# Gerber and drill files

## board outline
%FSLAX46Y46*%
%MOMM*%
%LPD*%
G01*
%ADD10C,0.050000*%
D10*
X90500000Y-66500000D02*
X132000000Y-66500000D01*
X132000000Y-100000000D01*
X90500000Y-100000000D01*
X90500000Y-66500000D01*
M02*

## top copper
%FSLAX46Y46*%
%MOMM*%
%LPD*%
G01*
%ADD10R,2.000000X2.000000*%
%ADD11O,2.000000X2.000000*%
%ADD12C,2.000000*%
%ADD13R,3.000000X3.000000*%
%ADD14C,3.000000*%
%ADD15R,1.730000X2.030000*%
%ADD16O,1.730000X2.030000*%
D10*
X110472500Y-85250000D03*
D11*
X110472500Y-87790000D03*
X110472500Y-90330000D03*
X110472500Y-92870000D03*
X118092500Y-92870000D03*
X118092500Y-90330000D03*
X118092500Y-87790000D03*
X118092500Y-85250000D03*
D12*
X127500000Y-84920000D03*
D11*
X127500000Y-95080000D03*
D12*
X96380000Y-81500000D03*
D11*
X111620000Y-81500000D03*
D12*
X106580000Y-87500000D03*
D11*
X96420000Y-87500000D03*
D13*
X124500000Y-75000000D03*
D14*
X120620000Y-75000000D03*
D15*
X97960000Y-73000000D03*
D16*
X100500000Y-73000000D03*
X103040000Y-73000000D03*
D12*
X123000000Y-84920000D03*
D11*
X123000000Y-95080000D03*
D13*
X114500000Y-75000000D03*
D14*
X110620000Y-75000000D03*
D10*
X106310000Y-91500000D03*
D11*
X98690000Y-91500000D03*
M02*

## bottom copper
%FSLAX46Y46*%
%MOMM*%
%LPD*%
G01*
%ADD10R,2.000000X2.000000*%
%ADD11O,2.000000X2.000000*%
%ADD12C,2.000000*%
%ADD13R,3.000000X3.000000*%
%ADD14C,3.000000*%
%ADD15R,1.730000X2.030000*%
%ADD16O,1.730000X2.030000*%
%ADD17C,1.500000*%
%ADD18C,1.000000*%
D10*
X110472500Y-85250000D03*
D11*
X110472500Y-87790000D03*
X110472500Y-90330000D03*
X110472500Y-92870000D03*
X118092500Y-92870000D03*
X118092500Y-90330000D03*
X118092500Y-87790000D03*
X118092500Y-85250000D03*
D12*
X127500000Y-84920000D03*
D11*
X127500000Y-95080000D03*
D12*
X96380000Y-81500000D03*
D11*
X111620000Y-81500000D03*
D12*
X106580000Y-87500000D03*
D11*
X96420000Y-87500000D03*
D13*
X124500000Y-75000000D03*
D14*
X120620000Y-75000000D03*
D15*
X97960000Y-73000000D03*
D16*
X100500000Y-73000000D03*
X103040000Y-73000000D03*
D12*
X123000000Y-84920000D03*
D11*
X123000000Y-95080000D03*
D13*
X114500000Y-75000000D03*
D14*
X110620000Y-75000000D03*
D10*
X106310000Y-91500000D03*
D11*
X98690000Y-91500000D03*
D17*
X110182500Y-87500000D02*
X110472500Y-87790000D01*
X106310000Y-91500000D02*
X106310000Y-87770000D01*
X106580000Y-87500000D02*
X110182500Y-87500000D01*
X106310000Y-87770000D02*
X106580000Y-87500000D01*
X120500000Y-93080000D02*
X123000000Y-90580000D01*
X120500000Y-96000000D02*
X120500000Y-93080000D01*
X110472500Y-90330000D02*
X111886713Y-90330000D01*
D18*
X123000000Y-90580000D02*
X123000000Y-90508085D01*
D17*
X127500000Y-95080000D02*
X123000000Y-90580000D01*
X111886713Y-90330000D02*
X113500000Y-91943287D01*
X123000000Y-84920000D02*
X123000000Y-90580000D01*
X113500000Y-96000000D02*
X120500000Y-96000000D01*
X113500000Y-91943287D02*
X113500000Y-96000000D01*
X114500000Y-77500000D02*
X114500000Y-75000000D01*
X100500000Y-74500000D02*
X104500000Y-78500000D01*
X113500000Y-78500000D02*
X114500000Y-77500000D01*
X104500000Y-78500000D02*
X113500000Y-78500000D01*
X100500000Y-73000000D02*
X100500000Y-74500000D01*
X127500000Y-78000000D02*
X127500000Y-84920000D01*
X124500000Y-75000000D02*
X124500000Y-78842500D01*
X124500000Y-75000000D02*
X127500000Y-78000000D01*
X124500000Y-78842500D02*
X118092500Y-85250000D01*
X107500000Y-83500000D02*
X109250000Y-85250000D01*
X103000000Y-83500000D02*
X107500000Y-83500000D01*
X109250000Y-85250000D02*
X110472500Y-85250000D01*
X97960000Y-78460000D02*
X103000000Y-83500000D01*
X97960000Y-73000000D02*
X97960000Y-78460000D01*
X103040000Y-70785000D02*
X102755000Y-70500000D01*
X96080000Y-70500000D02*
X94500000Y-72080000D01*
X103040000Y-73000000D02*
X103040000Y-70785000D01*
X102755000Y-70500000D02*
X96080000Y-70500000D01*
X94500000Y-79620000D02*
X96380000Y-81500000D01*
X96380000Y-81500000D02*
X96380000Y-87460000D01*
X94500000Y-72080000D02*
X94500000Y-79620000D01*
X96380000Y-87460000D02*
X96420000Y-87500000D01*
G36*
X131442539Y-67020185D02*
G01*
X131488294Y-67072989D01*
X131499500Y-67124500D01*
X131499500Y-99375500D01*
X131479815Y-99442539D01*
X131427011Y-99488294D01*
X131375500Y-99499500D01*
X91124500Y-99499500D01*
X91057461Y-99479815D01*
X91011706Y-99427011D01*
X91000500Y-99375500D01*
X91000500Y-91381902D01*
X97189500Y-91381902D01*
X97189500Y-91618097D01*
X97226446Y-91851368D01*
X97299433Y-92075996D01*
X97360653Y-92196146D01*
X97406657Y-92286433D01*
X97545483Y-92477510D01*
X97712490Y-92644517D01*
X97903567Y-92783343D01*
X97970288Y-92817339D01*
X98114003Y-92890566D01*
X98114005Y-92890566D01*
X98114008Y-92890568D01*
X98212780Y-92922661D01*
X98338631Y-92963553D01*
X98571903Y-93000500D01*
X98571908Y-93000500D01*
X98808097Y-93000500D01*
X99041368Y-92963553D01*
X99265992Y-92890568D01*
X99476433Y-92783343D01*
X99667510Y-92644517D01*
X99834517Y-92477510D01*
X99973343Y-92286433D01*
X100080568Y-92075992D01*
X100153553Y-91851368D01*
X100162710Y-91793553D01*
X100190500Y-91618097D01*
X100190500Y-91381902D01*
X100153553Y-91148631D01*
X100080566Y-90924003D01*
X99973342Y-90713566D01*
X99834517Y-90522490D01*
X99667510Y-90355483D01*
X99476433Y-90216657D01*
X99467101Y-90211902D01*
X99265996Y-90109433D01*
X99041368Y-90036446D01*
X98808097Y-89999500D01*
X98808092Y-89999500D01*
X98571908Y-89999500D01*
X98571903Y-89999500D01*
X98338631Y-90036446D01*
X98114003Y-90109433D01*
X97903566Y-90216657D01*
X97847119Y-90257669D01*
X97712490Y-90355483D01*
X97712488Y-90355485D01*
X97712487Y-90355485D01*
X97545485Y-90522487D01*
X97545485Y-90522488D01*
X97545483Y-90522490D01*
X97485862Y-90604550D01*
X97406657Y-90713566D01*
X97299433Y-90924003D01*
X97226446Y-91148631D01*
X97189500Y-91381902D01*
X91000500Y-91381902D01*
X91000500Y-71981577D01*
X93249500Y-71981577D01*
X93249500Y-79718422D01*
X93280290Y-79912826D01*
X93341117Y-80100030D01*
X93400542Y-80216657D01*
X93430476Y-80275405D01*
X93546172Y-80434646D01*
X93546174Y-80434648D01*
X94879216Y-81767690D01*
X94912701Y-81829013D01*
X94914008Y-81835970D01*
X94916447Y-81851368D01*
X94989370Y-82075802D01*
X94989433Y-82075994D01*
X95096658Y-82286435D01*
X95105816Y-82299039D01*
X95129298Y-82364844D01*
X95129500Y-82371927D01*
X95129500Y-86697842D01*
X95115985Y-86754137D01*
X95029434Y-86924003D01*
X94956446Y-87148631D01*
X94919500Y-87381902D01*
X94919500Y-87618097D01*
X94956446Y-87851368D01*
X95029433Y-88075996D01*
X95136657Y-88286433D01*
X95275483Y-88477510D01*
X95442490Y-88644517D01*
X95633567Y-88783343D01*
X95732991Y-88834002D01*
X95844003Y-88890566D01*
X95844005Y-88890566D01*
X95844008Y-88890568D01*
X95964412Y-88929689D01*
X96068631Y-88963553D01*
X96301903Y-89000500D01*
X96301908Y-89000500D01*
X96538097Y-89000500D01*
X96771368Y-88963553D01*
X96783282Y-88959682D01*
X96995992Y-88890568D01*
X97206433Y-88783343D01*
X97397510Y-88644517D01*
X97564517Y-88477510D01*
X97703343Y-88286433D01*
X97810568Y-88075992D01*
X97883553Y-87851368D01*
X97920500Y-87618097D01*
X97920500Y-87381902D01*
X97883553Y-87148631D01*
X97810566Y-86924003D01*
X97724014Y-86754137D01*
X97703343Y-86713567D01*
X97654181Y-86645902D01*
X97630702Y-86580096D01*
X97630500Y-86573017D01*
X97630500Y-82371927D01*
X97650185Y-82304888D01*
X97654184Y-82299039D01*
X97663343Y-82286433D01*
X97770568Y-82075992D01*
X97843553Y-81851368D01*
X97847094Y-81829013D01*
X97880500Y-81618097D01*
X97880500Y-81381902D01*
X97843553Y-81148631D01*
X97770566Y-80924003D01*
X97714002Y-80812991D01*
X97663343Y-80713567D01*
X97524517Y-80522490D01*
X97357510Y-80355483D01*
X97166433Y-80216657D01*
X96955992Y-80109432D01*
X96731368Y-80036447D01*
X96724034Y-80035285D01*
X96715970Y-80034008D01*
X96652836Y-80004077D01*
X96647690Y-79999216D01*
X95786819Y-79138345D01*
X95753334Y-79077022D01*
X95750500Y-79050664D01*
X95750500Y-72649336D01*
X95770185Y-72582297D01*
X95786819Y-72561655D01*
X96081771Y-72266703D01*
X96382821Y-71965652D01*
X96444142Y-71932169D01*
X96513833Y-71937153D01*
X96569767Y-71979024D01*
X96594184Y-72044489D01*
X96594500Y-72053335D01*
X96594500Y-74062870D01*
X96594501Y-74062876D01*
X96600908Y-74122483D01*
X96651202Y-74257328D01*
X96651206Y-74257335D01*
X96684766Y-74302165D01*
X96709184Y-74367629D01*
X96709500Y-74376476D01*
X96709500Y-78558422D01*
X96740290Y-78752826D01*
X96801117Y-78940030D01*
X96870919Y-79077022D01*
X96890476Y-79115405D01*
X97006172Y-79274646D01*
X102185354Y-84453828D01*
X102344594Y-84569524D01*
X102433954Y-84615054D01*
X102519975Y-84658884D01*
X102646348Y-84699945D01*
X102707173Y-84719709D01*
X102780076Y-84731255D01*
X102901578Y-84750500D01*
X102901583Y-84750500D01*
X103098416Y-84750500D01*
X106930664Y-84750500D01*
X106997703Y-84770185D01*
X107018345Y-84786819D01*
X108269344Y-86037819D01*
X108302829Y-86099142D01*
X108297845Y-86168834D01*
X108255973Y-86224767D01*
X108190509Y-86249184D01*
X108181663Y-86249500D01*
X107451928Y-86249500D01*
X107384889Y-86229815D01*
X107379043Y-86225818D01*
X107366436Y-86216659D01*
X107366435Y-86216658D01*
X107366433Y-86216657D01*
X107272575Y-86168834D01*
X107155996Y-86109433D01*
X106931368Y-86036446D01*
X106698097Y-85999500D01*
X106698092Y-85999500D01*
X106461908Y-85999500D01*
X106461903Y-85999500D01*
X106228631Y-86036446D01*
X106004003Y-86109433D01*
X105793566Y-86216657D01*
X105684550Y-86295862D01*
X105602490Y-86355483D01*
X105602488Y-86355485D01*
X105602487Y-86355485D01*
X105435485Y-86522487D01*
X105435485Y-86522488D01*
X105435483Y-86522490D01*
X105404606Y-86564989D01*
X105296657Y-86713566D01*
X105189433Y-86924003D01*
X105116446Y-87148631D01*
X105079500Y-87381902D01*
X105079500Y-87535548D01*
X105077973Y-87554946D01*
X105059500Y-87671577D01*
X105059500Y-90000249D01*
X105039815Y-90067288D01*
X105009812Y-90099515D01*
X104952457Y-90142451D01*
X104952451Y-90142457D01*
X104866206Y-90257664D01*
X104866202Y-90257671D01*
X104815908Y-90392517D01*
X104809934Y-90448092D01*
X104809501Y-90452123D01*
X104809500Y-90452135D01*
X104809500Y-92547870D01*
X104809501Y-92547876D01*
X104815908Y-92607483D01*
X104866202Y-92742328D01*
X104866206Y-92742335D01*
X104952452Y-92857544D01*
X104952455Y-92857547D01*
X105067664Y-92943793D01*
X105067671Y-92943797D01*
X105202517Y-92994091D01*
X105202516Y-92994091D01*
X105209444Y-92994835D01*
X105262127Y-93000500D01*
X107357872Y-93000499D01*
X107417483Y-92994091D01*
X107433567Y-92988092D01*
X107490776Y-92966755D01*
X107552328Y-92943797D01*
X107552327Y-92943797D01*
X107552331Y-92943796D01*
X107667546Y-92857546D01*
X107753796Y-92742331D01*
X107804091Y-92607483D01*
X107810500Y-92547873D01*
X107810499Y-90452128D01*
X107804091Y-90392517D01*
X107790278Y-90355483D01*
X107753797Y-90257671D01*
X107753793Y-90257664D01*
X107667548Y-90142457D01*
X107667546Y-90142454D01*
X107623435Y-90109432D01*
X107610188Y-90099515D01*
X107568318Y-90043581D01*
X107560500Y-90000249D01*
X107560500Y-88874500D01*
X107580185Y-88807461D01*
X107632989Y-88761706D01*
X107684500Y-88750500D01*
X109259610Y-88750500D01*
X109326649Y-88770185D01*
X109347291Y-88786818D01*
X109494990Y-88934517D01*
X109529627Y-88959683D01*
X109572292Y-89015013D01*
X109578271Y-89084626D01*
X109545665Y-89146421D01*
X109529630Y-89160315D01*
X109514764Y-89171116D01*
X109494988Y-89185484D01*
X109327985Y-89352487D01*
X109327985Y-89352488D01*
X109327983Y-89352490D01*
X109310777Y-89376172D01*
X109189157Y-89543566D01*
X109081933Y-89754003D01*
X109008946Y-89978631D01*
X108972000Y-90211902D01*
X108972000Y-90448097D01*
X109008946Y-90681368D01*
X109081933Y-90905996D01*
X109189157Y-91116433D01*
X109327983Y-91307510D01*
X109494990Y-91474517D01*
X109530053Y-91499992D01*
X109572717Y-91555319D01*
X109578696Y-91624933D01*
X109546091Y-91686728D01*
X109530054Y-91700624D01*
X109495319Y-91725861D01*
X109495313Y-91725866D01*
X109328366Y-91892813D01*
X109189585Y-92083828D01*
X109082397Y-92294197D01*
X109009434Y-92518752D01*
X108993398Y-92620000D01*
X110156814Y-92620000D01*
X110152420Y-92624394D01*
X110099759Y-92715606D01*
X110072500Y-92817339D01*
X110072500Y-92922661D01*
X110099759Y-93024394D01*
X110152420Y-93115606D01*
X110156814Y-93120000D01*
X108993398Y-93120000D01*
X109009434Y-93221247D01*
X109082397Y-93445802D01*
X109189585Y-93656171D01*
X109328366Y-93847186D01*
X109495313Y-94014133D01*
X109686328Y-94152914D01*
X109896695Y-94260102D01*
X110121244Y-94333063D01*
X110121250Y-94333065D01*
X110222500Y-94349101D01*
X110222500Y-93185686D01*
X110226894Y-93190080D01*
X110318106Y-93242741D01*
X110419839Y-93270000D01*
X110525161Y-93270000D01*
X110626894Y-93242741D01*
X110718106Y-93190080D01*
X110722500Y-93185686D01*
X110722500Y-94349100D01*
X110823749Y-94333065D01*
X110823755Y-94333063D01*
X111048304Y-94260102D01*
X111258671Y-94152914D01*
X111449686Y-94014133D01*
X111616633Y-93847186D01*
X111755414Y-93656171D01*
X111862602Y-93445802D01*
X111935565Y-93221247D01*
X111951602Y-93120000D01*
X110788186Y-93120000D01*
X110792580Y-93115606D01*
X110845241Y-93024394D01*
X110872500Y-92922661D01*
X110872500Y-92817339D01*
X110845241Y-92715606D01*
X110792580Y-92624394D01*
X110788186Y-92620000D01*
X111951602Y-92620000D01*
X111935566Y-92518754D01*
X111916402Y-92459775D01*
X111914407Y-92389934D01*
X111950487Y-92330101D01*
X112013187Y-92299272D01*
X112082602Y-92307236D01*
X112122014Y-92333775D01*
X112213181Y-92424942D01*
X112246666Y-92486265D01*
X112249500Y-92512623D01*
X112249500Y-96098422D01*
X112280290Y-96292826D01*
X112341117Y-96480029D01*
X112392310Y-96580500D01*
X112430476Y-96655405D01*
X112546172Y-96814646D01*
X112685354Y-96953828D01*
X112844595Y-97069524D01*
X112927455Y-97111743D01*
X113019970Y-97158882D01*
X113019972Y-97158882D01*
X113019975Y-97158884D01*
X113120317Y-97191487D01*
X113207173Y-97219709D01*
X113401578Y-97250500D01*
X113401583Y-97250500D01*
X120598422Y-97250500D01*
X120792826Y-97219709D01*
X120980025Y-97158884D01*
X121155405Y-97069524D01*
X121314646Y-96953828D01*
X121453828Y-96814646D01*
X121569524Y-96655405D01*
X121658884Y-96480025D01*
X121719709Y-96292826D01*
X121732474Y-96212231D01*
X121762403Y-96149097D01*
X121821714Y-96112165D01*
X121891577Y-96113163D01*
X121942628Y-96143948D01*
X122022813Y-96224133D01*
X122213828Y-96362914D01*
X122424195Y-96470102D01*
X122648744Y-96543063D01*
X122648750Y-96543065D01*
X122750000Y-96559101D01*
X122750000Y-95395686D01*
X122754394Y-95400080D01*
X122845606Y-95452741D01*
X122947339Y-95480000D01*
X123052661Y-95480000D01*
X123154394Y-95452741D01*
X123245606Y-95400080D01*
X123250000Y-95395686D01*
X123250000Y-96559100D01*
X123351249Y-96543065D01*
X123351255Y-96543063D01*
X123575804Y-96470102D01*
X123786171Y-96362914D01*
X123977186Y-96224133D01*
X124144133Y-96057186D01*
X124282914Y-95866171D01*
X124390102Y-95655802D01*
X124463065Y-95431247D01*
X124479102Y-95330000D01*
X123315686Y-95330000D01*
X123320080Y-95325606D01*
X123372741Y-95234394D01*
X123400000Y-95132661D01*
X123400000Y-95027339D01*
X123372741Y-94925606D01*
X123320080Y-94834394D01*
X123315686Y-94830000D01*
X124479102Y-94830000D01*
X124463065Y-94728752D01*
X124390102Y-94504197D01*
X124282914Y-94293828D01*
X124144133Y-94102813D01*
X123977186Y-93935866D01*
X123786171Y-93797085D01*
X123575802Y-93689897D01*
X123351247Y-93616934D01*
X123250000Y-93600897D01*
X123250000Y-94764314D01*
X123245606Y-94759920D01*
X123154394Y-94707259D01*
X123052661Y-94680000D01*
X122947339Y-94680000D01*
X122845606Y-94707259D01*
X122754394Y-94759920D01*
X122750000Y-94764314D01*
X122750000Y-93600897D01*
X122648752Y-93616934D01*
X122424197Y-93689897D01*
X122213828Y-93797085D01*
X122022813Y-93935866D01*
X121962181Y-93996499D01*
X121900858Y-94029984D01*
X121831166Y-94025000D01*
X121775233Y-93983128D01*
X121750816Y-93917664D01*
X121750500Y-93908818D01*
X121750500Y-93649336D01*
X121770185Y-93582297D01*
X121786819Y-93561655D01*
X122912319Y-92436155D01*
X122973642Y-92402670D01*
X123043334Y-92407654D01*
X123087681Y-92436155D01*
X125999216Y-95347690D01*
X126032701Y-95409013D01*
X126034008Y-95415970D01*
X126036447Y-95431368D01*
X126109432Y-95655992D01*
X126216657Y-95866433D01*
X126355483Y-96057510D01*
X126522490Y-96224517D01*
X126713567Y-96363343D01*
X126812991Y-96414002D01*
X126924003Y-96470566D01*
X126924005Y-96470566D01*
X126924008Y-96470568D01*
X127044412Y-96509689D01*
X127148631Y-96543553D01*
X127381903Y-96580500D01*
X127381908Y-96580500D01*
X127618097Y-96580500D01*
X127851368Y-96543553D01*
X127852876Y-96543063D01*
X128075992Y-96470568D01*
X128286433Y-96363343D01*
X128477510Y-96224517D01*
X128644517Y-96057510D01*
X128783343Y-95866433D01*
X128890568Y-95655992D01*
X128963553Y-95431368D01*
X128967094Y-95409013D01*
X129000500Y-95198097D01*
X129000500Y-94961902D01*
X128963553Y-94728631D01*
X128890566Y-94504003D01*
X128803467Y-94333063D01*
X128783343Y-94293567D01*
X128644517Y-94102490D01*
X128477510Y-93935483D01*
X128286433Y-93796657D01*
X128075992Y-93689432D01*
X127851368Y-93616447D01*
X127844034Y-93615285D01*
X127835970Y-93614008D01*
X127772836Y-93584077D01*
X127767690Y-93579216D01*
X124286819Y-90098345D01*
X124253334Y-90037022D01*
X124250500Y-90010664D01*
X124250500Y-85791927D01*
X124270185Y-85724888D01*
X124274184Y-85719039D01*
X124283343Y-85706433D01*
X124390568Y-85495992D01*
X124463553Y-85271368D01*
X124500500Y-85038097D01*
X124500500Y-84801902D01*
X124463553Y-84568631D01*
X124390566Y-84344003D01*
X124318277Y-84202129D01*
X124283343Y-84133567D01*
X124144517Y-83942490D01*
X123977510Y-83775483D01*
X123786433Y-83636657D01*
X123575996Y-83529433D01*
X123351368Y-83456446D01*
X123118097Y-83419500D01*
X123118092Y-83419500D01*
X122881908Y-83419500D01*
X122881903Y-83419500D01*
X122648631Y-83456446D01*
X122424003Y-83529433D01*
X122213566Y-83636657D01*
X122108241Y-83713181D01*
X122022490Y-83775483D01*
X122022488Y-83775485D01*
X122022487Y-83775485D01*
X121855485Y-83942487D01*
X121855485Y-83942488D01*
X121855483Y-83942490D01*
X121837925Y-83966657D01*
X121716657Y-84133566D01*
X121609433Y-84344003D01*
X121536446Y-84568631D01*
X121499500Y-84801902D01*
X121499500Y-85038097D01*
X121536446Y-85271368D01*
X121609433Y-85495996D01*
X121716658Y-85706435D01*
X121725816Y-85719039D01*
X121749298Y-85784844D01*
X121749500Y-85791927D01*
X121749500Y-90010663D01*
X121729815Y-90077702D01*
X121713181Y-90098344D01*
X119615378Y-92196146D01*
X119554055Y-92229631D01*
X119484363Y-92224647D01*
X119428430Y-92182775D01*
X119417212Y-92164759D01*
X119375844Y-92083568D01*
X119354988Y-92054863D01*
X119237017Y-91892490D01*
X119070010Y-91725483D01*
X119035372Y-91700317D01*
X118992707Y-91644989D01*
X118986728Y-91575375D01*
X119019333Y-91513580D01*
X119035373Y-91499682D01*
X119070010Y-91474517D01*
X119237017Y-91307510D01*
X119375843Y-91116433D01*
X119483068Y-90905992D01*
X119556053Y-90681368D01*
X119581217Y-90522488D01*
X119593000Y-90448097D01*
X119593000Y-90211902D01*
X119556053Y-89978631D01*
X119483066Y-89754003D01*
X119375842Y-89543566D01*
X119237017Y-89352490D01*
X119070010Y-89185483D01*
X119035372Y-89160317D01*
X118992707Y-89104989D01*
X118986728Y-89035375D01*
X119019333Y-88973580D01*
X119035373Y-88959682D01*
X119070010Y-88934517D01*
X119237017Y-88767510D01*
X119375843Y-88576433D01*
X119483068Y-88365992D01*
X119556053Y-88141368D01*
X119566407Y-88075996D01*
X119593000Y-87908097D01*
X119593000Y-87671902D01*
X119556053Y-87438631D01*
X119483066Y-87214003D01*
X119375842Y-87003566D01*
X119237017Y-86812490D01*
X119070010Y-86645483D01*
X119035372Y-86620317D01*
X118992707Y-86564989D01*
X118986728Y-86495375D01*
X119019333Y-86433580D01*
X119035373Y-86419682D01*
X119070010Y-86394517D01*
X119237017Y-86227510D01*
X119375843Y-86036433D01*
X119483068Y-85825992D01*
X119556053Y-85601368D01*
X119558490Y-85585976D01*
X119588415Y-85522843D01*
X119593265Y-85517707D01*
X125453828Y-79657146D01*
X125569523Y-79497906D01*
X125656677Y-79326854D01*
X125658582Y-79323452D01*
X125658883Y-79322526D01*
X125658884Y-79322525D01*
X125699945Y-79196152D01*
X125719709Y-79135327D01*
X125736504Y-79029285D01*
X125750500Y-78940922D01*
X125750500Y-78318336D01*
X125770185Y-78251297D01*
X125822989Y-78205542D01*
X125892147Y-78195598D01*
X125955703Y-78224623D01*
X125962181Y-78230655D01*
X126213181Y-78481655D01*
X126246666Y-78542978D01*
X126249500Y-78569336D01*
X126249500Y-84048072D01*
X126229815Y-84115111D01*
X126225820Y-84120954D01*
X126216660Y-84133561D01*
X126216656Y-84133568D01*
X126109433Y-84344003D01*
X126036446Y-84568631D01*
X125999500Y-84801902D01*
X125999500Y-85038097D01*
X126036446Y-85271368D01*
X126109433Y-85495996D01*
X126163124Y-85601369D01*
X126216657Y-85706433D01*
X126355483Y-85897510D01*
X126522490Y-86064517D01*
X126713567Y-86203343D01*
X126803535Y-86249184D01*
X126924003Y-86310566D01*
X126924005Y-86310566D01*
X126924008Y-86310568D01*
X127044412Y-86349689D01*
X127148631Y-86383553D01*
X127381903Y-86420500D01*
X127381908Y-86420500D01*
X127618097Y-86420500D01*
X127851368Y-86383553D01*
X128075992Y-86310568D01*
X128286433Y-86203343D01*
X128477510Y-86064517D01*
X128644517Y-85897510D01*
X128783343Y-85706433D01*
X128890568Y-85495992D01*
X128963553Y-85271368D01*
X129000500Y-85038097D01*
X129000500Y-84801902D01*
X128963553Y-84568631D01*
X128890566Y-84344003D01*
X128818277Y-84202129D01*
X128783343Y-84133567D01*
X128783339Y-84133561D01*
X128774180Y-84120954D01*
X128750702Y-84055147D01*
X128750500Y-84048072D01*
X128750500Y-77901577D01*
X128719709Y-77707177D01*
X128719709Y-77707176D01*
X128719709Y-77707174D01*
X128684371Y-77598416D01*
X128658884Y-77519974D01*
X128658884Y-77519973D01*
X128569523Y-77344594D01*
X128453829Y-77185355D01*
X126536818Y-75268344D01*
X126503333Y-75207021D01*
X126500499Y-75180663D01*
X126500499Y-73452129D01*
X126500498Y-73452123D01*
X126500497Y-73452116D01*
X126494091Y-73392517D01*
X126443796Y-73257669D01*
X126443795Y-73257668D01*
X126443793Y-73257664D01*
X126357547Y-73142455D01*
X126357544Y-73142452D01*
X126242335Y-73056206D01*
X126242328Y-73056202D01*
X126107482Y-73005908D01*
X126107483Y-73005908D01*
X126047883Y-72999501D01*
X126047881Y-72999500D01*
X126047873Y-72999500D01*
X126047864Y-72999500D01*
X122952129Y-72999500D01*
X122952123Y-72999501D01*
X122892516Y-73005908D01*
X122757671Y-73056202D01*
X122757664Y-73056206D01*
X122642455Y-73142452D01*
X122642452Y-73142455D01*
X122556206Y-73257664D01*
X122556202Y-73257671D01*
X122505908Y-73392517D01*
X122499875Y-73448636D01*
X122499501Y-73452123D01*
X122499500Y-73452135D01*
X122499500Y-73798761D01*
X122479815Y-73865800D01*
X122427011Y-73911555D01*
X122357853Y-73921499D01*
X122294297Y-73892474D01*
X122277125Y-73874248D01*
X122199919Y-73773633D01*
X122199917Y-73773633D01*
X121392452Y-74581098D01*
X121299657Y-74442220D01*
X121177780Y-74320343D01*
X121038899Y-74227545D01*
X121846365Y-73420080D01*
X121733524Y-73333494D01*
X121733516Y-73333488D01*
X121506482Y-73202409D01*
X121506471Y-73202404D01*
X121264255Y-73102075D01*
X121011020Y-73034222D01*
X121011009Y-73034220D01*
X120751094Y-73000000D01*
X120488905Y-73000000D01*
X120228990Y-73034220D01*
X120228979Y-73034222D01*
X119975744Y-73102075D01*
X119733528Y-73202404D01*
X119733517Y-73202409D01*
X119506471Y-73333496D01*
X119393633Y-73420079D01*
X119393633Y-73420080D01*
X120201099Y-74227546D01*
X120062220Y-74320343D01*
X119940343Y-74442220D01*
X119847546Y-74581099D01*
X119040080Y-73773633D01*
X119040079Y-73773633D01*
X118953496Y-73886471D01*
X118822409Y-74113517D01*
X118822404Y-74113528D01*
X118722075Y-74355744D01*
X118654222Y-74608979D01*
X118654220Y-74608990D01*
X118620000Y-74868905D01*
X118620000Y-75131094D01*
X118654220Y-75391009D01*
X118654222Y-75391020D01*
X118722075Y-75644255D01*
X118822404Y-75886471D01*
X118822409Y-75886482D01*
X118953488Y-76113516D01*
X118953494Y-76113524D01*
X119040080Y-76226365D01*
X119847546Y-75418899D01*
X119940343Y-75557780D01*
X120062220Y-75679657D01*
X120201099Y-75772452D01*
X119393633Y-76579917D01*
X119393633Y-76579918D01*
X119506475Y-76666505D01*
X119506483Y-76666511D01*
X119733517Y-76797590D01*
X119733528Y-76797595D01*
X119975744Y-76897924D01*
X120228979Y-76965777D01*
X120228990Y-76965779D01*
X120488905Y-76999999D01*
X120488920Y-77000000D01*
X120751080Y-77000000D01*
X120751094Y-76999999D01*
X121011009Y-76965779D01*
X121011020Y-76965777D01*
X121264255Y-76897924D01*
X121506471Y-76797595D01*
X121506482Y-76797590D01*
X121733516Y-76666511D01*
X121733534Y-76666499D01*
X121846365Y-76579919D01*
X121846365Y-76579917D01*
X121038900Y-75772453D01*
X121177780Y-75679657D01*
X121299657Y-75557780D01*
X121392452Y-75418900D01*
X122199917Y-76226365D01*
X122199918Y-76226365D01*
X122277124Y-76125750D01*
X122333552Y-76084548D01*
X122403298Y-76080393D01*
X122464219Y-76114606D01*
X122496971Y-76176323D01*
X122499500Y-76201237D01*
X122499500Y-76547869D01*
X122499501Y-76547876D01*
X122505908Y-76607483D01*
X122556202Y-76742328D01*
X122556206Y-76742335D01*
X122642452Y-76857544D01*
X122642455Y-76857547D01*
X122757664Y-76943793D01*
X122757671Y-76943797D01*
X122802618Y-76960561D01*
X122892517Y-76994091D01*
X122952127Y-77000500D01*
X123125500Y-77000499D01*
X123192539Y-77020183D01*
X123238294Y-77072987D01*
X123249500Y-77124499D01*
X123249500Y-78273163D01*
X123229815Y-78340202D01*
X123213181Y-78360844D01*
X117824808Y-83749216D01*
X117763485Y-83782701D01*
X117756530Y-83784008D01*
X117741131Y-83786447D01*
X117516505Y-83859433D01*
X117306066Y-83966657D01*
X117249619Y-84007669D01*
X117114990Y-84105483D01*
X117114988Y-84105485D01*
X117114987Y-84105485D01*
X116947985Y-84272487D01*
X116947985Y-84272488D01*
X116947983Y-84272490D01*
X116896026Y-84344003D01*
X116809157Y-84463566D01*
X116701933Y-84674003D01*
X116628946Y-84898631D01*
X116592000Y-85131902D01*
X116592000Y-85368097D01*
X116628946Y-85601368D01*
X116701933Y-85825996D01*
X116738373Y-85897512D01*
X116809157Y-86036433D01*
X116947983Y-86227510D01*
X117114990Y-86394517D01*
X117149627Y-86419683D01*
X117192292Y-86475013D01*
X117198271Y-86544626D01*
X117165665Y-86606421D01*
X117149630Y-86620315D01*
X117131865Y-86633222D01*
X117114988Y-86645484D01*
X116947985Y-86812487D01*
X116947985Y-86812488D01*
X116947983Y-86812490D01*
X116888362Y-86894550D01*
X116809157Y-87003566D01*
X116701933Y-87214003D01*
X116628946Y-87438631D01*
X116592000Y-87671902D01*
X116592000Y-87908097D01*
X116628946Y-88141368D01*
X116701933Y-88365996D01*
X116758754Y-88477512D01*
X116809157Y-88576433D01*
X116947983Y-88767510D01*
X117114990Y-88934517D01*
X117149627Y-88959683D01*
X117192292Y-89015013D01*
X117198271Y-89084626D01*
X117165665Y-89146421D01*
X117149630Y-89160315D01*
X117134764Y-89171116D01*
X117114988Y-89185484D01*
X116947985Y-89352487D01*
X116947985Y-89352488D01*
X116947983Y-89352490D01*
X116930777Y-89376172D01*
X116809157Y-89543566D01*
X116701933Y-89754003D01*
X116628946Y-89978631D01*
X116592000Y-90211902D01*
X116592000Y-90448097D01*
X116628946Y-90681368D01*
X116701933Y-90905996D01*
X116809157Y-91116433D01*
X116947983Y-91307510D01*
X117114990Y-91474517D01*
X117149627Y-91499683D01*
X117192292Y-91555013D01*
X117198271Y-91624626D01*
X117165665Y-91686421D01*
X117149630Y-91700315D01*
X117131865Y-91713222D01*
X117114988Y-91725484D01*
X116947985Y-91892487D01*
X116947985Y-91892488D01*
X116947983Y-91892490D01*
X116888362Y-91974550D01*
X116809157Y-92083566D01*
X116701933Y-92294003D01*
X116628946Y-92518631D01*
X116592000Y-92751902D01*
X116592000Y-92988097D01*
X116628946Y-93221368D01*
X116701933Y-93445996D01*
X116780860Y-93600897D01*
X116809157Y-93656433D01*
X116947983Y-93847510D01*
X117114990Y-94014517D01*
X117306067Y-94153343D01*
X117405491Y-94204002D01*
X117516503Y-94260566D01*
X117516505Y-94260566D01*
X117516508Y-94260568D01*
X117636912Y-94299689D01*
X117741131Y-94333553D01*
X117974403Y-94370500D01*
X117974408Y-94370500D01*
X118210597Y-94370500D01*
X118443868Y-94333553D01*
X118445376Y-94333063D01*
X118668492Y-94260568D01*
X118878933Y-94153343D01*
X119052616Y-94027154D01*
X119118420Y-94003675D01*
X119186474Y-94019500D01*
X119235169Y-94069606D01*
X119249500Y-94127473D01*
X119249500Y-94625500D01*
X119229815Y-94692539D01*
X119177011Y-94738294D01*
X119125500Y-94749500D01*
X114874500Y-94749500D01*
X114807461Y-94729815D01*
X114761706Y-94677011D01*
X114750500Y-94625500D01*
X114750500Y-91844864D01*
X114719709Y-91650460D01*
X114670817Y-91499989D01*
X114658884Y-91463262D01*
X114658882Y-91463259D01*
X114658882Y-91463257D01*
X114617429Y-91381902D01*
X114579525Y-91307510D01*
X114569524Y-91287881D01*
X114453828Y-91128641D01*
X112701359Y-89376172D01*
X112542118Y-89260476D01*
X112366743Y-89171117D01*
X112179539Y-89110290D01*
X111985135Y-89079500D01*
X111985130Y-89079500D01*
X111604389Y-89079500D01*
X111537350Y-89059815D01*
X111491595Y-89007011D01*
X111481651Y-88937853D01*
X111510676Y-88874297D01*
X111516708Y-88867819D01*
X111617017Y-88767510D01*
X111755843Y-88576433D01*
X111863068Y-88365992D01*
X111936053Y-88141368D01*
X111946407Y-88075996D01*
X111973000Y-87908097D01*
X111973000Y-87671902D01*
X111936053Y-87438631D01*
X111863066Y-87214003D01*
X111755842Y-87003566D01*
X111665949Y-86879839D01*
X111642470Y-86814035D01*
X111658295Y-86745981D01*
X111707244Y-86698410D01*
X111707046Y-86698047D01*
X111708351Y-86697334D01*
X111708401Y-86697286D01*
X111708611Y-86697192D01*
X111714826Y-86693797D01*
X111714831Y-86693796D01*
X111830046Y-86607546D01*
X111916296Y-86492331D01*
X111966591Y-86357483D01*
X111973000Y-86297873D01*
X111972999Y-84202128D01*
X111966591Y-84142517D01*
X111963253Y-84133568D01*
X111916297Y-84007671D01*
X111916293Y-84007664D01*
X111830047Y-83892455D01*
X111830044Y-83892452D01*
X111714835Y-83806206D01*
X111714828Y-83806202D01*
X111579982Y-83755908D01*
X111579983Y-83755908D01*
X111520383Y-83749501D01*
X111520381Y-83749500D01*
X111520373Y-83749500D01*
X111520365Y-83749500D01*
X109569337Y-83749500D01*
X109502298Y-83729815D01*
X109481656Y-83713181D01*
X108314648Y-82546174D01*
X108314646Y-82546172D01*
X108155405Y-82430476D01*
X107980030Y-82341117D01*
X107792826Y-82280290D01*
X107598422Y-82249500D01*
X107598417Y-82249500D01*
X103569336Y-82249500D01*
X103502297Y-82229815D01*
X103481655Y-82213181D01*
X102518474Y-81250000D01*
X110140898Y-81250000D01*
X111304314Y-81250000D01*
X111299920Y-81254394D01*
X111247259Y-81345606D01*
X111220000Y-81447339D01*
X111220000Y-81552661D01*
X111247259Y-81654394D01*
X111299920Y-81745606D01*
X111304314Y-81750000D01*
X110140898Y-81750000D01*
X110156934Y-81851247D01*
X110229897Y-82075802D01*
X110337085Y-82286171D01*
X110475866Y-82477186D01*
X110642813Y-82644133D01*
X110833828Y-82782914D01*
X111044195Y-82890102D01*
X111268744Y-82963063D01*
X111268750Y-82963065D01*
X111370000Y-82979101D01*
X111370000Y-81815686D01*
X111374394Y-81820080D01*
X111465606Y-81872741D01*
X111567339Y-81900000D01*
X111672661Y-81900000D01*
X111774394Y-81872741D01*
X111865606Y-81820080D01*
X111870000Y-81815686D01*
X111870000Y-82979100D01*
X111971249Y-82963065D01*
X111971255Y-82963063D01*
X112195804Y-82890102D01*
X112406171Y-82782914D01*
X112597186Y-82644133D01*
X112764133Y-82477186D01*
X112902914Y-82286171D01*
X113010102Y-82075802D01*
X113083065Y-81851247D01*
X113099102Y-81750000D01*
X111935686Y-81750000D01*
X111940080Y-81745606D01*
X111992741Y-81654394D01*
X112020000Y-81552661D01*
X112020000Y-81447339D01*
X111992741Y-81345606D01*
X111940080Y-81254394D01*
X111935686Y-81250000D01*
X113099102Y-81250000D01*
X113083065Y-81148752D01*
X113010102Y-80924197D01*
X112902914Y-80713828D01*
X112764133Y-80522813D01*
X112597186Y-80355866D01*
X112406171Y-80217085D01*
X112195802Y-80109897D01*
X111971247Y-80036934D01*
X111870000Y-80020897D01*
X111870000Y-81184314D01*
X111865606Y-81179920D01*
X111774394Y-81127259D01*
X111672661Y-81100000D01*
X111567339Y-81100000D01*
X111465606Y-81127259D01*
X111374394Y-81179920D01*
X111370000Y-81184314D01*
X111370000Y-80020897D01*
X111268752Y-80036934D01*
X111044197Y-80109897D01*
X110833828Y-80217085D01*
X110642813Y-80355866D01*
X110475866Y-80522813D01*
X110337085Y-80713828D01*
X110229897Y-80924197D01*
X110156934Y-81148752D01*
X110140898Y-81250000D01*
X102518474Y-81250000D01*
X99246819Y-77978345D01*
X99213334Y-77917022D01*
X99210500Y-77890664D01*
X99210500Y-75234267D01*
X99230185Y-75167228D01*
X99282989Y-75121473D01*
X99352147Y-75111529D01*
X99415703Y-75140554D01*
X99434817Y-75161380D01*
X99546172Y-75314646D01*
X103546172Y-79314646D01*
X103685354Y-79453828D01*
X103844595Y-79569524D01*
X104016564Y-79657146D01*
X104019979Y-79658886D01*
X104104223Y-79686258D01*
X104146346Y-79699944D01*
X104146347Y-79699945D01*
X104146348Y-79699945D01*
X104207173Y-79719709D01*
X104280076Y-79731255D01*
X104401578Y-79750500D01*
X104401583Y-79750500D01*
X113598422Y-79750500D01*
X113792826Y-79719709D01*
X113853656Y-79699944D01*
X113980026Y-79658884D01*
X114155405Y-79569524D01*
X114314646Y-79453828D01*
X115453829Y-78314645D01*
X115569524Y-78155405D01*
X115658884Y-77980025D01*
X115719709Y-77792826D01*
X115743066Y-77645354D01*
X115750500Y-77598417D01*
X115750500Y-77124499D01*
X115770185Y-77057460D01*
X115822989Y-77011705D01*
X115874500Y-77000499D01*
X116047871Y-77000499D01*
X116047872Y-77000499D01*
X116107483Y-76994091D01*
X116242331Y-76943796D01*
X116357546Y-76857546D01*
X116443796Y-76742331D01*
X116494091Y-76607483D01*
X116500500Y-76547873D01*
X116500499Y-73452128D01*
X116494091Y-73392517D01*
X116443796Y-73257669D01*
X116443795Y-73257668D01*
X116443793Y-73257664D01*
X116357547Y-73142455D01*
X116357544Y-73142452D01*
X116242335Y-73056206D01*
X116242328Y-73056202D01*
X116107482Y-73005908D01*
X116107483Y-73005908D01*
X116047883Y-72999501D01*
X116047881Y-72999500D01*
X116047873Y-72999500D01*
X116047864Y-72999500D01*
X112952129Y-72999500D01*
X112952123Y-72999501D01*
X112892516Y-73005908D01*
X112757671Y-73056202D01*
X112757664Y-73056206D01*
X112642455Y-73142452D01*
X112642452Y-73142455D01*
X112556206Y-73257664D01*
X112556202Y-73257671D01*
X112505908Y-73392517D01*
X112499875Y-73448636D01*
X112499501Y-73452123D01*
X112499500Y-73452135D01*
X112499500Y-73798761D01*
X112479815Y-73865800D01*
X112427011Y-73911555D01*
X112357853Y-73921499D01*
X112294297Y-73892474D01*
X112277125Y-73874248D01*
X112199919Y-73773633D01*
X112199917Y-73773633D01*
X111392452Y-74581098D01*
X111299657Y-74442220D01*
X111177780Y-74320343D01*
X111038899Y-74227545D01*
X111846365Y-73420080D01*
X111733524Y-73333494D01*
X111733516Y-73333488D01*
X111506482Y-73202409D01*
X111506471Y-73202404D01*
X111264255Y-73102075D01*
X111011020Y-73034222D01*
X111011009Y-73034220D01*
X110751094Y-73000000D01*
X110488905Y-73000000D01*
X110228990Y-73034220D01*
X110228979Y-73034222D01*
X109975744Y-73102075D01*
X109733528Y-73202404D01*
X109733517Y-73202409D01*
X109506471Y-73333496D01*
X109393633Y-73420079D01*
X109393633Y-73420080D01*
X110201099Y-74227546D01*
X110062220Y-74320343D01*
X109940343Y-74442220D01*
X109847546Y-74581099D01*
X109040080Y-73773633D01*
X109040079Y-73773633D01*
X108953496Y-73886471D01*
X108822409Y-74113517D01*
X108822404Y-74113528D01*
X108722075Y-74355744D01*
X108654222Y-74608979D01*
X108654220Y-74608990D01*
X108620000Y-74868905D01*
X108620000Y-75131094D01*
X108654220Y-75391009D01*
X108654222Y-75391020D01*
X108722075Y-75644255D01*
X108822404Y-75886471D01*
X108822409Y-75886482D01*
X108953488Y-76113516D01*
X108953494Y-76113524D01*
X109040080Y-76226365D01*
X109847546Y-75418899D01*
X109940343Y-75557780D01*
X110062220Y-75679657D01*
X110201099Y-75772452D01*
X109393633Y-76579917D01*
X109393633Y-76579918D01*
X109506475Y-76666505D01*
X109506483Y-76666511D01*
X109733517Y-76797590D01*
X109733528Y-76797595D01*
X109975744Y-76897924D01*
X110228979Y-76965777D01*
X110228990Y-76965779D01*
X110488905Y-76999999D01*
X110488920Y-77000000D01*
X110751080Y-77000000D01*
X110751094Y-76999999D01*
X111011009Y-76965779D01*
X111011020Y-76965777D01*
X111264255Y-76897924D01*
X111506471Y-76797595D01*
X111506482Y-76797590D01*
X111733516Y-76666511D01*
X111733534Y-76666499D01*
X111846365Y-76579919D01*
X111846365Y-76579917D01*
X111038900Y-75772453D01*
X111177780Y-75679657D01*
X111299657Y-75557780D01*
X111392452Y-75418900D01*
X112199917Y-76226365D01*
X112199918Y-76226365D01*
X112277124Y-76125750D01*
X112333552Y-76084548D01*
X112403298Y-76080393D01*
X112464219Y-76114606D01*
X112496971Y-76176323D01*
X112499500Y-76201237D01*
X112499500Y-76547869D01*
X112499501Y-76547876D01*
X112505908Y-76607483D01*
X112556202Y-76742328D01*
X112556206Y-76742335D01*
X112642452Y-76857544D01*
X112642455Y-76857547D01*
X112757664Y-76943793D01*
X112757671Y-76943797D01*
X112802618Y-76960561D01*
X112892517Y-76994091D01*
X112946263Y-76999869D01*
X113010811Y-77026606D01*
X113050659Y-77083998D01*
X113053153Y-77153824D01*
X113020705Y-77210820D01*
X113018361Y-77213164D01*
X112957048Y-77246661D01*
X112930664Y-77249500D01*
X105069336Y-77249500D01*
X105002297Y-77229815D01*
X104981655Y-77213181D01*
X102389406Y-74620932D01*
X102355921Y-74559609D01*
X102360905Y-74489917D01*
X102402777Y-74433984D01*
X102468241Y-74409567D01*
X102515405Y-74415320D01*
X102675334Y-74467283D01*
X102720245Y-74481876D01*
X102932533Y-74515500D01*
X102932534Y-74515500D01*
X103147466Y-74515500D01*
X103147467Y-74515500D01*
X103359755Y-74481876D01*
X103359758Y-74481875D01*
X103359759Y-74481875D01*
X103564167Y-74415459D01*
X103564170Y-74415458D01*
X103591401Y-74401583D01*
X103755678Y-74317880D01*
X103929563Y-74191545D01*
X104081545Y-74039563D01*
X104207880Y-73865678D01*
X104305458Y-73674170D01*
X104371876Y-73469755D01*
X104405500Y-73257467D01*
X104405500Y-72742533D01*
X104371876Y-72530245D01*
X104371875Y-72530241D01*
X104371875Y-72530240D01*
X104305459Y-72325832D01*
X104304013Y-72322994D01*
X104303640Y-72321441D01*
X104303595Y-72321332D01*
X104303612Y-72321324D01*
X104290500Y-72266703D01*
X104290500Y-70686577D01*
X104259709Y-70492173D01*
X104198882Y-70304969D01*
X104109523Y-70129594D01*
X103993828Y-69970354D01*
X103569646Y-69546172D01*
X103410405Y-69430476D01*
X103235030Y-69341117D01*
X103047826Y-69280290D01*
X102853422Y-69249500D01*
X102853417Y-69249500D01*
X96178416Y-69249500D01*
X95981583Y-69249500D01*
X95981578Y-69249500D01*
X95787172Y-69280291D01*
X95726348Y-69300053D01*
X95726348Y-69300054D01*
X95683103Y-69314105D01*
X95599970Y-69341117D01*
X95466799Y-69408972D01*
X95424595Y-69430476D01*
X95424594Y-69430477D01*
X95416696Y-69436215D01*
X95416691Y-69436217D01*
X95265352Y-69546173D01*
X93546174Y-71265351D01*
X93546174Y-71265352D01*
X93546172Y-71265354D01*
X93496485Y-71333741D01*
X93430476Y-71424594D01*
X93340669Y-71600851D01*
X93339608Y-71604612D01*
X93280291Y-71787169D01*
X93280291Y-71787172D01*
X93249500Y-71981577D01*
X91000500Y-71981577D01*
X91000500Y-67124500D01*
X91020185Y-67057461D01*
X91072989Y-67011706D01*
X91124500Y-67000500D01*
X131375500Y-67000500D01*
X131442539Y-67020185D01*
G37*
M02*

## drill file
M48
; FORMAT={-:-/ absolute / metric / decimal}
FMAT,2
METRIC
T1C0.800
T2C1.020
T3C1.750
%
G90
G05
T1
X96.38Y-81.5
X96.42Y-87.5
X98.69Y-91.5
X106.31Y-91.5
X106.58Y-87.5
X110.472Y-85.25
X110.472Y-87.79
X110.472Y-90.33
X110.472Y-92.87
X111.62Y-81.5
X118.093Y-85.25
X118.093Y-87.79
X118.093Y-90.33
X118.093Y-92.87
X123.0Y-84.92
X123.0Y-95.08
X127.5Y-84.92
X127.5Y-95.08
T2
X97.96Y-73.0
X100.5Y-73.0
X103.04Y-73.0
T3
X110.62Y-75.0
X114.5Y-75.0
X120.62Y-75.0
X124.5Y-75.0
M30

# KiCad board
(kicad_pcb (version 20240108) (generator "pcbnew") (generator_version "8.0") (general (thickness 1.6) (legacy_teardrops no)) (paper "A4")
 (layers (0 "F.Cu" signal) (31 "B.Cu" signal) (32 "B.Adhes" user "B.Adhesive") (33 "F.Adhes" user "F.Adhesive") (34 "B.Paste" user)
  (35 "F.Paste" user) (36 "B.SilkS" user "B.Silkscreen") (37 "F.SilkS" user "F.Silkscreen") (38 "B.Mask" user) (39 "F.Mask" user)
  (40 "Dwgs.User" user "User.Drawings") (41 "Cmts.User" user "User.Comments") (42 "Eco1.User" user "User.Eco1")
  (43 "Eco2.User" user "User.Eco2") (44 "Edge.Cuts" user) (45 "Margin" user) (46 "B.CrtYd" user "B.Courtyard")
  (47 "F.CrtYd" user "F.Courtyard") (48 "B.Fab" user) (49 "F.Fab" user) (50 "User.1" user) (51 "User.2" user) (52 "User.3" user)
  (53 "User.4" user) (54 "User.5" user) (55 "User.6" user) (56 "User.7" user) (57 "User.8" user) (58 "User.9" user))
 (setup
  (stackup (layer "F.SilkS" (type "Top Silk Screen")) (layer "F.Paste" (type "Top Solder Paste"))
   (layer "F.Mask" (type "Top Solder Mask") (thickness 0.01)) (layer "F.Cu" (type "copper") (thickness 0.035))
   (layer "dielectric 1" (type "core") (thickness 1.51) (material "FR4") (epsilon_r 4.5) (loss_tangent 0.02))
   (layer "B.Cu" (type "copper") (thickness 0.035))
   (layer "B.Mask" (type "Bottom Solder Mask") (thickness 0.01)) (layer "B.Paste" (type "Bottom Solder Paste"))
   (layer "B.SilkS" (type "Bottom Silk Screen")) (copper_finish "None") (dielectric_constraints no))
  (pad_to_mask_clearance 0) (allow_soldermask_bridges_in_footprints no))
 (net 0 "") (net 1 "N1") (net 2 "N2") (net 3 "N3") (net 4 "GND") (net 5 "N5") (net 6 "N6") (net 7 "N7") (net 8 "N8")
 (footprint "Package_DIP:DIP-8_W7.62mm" (layer "F.Cu") (at 110.4725 85.25)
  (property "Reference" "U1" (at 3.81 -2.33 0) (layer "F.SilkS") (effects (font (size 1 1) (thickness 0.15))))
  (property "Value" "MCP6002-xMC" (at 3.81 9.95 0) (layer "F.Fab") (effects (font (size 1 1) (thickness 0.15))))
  (pad "1" thru_hole rect (at 0 0) (size 2 2) (drill 0.8) (layers "*.Cu" "*.Mask") (remove_unused_layers no) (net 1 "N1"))
  (pad "2" thru_hole oval (at 0 2.54) (size 2 2) (drill 0.8) (layers "*.Cu" "*.Mask") (remove_unused_layers no) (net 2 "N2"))
  (pad "3" thru_hole oval (at 0 5.08) (size 2 2) (drill 0.8) (layers "*.Cu" "*.Mask") (remove_unused_layers no) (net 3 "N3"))
  (pad "4" thru_hole oval (at 0 7.62) (size 2 2) (drill 0.8) (layers "*.Cu" "*.Mask") (remove_unused_layers no) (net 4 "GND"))
  (pad "5" thru_hole oval (at 7.62 7.62) (size 2 2) (drill 0.8) (layers "*.Cu" "*.Mask") (remove_unused_layers no))
  (pad "6" thru_hole oval (at 7.62 5.08) (size 2 2) (drill 0.8) (layers "*.Cu" "*.Mask") (remove_unused_layers no))
  (pad "7" thru_hole oval (at 7.62 2.54) (size 2 2) (drill 0.8) (layers "*.Cu" "*.Mask") (remove_unused_layers no))
  (pad "8" thru_hole oval (at 7.62 0) (size 2 2) (drill 0.8) (layers "*.Cu" "*.Mask") (remove_unused_layers no) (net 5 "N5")))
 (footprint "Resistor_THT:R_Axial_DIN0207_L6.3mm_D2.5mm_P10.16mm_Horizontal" (layer "F.Cu") (at 127.5 84.92 -90)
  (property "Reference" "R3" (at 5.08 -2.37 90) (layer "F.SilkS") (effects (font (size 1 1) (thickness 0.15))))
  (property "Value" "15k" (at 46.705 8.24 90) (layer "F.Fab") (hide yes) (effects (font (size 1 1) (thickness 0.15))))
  (pad "1" thru_hole circle (at 0 0 270) (size 2 2) (drill 0.8) (layers "*.Cu" "*.Mask") (remove_unused_layers no) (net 5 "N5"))
  (pad "2" thru_hole oval (at 10.16 0 270) (size 2 2) (drill 0.8) (layers "*.Cu" "*.Mask") (remove_unused_layers no) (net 3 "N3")))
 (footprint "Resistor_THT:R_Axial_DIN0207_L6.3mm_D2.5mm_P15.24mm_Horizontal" (layer "F.Cu") (at 96.38 81.5)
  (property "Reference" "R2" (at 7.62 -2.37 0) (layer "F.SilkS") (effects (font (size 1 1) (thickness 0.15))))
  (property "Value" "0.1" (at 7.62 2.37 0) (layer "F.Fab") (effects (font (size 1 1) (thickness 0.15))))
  (pad "1" thru_hole circle (at 0 0) (size 2 2) (drill 0.8) (layers "*.Cu" "*.Mask") (remove_unused_layers no) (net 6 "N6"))
  (pad "2" thru_hole oval (at 15.24 0) (size 2 2) (drill 0.8) (layers "*.Cu" "*.Mask") (remove_unused_layers no) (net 4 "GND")))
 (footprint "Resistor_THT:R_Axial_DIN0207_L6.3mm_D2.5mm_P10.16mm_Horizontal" (layer "F.Cu") (at 106.58 87.5 180)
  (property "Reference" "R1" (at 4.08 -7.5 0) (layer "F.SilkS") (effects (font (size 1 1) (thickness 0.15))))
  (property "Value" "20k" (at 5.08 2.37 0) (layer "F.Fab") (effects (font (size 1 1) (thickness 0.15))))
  (pad "1" thru_hole circle (at 0 0 180) (size 2 2) (drill 0.8) (layers "*.Cu" "*.Mask") (remove_unused_layers no) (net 2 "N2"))
  (pad "2" thru_hole oval (at 10.16 0 180) (size 2 2) (drill 0.8) (layers "*.Cu" "*.Mask") (remove_unused_layers no) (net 6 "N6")))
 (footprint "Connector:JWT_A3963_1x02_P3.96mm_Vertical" (layer "F.Cu") (at 124.5 75 180)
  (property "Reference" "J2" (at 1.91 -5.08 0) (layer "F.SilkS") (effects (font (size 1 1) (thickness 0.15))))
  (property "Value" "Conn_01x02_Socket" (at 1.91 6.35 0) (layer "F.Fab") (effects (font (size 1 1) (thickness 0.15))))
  (pad "1" thru_hole rect (at 0 0 180) (size 3 3) (drill 1.75) (layers "*.Cu" "*.Mask") (remove_unused_layers no) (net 5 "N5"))
  (pad "2" thru_hole circle (at 3.88 0 180) (size 3 3) (drill 1.75) (layers "*.Cu" "*.Mask") (remove_unused_layers no) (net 4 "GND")))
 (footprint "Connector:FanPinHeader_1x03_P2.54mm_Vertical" (layer "F.Cu") (at 97.96 73)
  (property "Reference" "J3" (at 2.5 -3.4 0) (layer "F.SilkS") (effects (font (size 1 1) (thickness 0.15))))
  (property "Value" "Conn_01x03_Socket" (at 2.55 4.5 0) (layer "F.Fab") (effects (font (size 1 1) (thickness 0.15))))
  (pad "1" thru_hole rect (at 0 0 90) (size 2.03 1.73) (drill 1.02) (layers "*.Cu" "*.Mask") (remove_unused_layers no) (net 1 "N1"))
  (pad "2" thru_hole oval (at 2.54 0 90) (size 2.03 1.73) (drill 1.02) (layers "*.Cu" "*.Mask") (remove_unused_layers no) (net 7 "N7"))
  (pad "3" thru_hole oval (at 5.08 0 90) (size 2.03 1.73) (drill 1.02) (layers "*.Cu" "*.Mask") (remove_unused_layers no) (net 6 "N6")))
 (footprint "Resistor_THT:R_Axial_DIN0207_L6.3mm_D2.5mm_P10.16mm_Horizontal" (layer "F.Cu") (at 123 84.92 -90)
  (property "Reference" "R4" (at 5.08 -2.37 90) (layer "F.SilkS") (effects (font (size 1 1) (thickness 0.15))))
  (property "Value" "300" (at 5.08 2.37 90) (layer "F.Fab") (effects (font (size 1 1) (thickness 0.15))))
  (pad "1" thru_hole circle (at 0 0 270) (size 2 2) (drill 0.8) (layers "*.Cu" "*.Mask") (remove_unused_layers no) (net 3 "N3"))
  (pad "2" thru_hole oval (at 10.16 0 270) (size 2 2) (drill 0.8) (layers "*.Cu" "*.Mask") (remove_unused_layers no) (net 4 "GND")))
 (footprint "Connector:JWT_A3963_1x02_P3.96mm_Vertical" (layer "F.Cu") (at 114.5 75 180)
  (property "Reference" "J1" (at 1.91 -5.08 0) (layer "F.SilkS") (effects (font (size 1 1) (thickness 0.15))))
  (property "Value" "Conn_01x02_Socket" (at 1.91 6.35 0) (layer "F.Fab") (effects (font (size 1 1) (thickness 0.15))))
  (pad "1" thru_hole rect (at 0 0 180) (size 3 3) (drill 1.75) (layers "*.Cu" "*.Mask") (remove_unused_layers no) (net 7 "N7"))
  (pad "2" thru_hole circle (at 3.88 0 180) (size 3 3) (drill 1.75) (layers "*.Cu" "*.Mask") (remove_unused_layers no) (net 4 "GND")))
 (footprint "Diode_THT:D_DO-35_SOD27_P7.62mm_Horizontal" (layer "F.Cu") (at 106.31 91.5 180)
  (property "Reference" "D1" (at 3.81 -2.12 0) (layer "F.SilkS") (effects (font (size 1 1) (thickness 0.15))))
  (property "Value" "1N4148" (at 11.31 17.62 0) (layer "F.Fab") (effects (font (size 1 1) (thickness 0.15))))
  (pad "1" thru_hole rect (at 0 0 180) (size 2 2) (drill 0.8) (layers "*.Cu" "*.Mask") (remove_unused_layers no) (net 2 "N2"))
  (pad "2" thru_hole oval (at 7.62 0 180) (size 2 2) (drill 0.8) (layers "*.Cu" "*.Mask") (remove_unused_layers no) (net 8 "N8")))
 (gr_rect (start 90.5 66.5) (end 132 100) (stroke (width 0.05) (type default)) (fill none) (layer "Edge.Cuts"))
 (segment (start 110.1825 87.5) (end 110.4725 87.79) (width 1.5) (layer "B.Cu") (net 2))
 (segment (start 106.31 91.5) (end 106.31 87.77) (width 1.5) (layer "B.Cu") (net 2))
 (segment (start 106.58 87.5) (end 110.1825 87.5) (width 1.5) (layer "B.Cu") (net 2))
 (segment (start 106.31 87.77) (end 106.58 87.5) (width 1.5) (layer "B.Cu") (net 2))
 (segment (start 120.5 93.08) (end 123 90.58) (width 1.5) (layer "B.Cu") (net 3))
 (segment (start 120.5 96) (end 120.5 93.08) (width 1.5) (layer "B.Cu") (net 3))
 (segment (start 110.4725 90.33) (end 111.886713 90.33) (width 1.5) (layer "B.Cu") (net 3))
 (segment (start 123 90.58) (end 123 90.508085) (width 1) (layer "B.Cu") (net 3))
 (segment (start 127.5 95.08) (end 123 90.58) (width 1.5) (layer "B.Cu") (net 3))
 (segment (start 111.886713 90.33) (end 113.5 91.943287) (width 1.5) (layer "B.Cu") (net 3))
 (segment (start 123 84.92) (end 123 90.58) (width 1.5) (layer "B.Cu") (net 3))
 (segment (start 113.5 96) (end 120.5 96) (width 1.5) (layer "B.Cu") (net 3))
 (segment (start 113.5 91.943287) (end 113.5 96) (width 1.5) (layer "B.Cu") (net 3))
 (segment (start 114.5 77.5) (end 114.5 75) (width 1.5) (layer "B.Cu") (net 7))
 (segment (start 100.5 74.5) (end 104.5 78.5) (width 1.5) (layer "B.Cu") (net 7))
 (segment (start 113.5 78.5) (end 114.5 77.5) (width 1.5) (layer "B.Cu") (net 7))
 (segment (start 104.5 78.5) (end 113.5 78.5) (width 1.5) (layer "B.Cu") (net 7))
 (segment (start 100.5 73) (end 100.5 74.5) (width 1.5) (layer "B.Cu") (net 7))
 (segment (start 127.5 78) (end 127.5 84.92) (width 1.5) (layer "B.Cu") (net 5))
 (segment (start 124.5 75) (end 124.5 78.8425) (width 1.5) (layer "B.Cu") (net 5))
 (segment (start 124.5 75) (end 127.5 78) (width 1.5) (layer "B.Cu") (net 5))
 (segment (start 124.5 78.8425) (end 118.0925 85.25) (width 1.5) (layer "B.Cu") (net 5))
 (segment (start 107.5 83.5) (end 109.25 85.25) (width 1.5) (layer "B.Cu") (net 1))
 (segment (start 103 83.5) (end 107.5 83.5) (width 1.5) (layer "B.Cu") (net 1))
 (segment (start 109.25 85.25) (end 110.4725 85.25) (width 1.5) (layer "B.Cu") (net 1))
 (segment (start 97.96 78.46) (end 103 83.5) (width 1.5) (layer "B.Cu") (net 1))
 (segment (start 97.96 73) (end 97.96 78.46) (width 1.5) (layer "B.Cu") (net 1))
 (segment (start 103.04 70.785) (end 102.755 70.5) (width 1.5) (layer "B.Cu") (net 6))
 (segment (start 96.08 70.5) (end 94.5 72.08) (width 1.5) (layer "B.Cu") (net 6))
 (segment (start 103.04 73) (end 103.04 70.785) (width 1.5) (layer "B.Cu") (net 6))
 (segment (start 102.755 70.5) (end 96.08 70.5) (width 1.5) (layer "B.Cu") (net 6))
 (segment (start 94.5 79.62) (end 96.38 81.5) (width 1.5) (layer "B.Cu") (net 6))
 (segment (start 96.38 81.5) (end 96.38 87.46) (width 1.5) (layer "B.Cu") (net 6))
 (segment (start 94.5 72.08) (end 94.5 79.62) (width 1.5) (layer "B.Cu") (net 6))
 (segment (start 96.38 87.46) (end 96.42 87.5) (width 1.5) (layer "B.Cu") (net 6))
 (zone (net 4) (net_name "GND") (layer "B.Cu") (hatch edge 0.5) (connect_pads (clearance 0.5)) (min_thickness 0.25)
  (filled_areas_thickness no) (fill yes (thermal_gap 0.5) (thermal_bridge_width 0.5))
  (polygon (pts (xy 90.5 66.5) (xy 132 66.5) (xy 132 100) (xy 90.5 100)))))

